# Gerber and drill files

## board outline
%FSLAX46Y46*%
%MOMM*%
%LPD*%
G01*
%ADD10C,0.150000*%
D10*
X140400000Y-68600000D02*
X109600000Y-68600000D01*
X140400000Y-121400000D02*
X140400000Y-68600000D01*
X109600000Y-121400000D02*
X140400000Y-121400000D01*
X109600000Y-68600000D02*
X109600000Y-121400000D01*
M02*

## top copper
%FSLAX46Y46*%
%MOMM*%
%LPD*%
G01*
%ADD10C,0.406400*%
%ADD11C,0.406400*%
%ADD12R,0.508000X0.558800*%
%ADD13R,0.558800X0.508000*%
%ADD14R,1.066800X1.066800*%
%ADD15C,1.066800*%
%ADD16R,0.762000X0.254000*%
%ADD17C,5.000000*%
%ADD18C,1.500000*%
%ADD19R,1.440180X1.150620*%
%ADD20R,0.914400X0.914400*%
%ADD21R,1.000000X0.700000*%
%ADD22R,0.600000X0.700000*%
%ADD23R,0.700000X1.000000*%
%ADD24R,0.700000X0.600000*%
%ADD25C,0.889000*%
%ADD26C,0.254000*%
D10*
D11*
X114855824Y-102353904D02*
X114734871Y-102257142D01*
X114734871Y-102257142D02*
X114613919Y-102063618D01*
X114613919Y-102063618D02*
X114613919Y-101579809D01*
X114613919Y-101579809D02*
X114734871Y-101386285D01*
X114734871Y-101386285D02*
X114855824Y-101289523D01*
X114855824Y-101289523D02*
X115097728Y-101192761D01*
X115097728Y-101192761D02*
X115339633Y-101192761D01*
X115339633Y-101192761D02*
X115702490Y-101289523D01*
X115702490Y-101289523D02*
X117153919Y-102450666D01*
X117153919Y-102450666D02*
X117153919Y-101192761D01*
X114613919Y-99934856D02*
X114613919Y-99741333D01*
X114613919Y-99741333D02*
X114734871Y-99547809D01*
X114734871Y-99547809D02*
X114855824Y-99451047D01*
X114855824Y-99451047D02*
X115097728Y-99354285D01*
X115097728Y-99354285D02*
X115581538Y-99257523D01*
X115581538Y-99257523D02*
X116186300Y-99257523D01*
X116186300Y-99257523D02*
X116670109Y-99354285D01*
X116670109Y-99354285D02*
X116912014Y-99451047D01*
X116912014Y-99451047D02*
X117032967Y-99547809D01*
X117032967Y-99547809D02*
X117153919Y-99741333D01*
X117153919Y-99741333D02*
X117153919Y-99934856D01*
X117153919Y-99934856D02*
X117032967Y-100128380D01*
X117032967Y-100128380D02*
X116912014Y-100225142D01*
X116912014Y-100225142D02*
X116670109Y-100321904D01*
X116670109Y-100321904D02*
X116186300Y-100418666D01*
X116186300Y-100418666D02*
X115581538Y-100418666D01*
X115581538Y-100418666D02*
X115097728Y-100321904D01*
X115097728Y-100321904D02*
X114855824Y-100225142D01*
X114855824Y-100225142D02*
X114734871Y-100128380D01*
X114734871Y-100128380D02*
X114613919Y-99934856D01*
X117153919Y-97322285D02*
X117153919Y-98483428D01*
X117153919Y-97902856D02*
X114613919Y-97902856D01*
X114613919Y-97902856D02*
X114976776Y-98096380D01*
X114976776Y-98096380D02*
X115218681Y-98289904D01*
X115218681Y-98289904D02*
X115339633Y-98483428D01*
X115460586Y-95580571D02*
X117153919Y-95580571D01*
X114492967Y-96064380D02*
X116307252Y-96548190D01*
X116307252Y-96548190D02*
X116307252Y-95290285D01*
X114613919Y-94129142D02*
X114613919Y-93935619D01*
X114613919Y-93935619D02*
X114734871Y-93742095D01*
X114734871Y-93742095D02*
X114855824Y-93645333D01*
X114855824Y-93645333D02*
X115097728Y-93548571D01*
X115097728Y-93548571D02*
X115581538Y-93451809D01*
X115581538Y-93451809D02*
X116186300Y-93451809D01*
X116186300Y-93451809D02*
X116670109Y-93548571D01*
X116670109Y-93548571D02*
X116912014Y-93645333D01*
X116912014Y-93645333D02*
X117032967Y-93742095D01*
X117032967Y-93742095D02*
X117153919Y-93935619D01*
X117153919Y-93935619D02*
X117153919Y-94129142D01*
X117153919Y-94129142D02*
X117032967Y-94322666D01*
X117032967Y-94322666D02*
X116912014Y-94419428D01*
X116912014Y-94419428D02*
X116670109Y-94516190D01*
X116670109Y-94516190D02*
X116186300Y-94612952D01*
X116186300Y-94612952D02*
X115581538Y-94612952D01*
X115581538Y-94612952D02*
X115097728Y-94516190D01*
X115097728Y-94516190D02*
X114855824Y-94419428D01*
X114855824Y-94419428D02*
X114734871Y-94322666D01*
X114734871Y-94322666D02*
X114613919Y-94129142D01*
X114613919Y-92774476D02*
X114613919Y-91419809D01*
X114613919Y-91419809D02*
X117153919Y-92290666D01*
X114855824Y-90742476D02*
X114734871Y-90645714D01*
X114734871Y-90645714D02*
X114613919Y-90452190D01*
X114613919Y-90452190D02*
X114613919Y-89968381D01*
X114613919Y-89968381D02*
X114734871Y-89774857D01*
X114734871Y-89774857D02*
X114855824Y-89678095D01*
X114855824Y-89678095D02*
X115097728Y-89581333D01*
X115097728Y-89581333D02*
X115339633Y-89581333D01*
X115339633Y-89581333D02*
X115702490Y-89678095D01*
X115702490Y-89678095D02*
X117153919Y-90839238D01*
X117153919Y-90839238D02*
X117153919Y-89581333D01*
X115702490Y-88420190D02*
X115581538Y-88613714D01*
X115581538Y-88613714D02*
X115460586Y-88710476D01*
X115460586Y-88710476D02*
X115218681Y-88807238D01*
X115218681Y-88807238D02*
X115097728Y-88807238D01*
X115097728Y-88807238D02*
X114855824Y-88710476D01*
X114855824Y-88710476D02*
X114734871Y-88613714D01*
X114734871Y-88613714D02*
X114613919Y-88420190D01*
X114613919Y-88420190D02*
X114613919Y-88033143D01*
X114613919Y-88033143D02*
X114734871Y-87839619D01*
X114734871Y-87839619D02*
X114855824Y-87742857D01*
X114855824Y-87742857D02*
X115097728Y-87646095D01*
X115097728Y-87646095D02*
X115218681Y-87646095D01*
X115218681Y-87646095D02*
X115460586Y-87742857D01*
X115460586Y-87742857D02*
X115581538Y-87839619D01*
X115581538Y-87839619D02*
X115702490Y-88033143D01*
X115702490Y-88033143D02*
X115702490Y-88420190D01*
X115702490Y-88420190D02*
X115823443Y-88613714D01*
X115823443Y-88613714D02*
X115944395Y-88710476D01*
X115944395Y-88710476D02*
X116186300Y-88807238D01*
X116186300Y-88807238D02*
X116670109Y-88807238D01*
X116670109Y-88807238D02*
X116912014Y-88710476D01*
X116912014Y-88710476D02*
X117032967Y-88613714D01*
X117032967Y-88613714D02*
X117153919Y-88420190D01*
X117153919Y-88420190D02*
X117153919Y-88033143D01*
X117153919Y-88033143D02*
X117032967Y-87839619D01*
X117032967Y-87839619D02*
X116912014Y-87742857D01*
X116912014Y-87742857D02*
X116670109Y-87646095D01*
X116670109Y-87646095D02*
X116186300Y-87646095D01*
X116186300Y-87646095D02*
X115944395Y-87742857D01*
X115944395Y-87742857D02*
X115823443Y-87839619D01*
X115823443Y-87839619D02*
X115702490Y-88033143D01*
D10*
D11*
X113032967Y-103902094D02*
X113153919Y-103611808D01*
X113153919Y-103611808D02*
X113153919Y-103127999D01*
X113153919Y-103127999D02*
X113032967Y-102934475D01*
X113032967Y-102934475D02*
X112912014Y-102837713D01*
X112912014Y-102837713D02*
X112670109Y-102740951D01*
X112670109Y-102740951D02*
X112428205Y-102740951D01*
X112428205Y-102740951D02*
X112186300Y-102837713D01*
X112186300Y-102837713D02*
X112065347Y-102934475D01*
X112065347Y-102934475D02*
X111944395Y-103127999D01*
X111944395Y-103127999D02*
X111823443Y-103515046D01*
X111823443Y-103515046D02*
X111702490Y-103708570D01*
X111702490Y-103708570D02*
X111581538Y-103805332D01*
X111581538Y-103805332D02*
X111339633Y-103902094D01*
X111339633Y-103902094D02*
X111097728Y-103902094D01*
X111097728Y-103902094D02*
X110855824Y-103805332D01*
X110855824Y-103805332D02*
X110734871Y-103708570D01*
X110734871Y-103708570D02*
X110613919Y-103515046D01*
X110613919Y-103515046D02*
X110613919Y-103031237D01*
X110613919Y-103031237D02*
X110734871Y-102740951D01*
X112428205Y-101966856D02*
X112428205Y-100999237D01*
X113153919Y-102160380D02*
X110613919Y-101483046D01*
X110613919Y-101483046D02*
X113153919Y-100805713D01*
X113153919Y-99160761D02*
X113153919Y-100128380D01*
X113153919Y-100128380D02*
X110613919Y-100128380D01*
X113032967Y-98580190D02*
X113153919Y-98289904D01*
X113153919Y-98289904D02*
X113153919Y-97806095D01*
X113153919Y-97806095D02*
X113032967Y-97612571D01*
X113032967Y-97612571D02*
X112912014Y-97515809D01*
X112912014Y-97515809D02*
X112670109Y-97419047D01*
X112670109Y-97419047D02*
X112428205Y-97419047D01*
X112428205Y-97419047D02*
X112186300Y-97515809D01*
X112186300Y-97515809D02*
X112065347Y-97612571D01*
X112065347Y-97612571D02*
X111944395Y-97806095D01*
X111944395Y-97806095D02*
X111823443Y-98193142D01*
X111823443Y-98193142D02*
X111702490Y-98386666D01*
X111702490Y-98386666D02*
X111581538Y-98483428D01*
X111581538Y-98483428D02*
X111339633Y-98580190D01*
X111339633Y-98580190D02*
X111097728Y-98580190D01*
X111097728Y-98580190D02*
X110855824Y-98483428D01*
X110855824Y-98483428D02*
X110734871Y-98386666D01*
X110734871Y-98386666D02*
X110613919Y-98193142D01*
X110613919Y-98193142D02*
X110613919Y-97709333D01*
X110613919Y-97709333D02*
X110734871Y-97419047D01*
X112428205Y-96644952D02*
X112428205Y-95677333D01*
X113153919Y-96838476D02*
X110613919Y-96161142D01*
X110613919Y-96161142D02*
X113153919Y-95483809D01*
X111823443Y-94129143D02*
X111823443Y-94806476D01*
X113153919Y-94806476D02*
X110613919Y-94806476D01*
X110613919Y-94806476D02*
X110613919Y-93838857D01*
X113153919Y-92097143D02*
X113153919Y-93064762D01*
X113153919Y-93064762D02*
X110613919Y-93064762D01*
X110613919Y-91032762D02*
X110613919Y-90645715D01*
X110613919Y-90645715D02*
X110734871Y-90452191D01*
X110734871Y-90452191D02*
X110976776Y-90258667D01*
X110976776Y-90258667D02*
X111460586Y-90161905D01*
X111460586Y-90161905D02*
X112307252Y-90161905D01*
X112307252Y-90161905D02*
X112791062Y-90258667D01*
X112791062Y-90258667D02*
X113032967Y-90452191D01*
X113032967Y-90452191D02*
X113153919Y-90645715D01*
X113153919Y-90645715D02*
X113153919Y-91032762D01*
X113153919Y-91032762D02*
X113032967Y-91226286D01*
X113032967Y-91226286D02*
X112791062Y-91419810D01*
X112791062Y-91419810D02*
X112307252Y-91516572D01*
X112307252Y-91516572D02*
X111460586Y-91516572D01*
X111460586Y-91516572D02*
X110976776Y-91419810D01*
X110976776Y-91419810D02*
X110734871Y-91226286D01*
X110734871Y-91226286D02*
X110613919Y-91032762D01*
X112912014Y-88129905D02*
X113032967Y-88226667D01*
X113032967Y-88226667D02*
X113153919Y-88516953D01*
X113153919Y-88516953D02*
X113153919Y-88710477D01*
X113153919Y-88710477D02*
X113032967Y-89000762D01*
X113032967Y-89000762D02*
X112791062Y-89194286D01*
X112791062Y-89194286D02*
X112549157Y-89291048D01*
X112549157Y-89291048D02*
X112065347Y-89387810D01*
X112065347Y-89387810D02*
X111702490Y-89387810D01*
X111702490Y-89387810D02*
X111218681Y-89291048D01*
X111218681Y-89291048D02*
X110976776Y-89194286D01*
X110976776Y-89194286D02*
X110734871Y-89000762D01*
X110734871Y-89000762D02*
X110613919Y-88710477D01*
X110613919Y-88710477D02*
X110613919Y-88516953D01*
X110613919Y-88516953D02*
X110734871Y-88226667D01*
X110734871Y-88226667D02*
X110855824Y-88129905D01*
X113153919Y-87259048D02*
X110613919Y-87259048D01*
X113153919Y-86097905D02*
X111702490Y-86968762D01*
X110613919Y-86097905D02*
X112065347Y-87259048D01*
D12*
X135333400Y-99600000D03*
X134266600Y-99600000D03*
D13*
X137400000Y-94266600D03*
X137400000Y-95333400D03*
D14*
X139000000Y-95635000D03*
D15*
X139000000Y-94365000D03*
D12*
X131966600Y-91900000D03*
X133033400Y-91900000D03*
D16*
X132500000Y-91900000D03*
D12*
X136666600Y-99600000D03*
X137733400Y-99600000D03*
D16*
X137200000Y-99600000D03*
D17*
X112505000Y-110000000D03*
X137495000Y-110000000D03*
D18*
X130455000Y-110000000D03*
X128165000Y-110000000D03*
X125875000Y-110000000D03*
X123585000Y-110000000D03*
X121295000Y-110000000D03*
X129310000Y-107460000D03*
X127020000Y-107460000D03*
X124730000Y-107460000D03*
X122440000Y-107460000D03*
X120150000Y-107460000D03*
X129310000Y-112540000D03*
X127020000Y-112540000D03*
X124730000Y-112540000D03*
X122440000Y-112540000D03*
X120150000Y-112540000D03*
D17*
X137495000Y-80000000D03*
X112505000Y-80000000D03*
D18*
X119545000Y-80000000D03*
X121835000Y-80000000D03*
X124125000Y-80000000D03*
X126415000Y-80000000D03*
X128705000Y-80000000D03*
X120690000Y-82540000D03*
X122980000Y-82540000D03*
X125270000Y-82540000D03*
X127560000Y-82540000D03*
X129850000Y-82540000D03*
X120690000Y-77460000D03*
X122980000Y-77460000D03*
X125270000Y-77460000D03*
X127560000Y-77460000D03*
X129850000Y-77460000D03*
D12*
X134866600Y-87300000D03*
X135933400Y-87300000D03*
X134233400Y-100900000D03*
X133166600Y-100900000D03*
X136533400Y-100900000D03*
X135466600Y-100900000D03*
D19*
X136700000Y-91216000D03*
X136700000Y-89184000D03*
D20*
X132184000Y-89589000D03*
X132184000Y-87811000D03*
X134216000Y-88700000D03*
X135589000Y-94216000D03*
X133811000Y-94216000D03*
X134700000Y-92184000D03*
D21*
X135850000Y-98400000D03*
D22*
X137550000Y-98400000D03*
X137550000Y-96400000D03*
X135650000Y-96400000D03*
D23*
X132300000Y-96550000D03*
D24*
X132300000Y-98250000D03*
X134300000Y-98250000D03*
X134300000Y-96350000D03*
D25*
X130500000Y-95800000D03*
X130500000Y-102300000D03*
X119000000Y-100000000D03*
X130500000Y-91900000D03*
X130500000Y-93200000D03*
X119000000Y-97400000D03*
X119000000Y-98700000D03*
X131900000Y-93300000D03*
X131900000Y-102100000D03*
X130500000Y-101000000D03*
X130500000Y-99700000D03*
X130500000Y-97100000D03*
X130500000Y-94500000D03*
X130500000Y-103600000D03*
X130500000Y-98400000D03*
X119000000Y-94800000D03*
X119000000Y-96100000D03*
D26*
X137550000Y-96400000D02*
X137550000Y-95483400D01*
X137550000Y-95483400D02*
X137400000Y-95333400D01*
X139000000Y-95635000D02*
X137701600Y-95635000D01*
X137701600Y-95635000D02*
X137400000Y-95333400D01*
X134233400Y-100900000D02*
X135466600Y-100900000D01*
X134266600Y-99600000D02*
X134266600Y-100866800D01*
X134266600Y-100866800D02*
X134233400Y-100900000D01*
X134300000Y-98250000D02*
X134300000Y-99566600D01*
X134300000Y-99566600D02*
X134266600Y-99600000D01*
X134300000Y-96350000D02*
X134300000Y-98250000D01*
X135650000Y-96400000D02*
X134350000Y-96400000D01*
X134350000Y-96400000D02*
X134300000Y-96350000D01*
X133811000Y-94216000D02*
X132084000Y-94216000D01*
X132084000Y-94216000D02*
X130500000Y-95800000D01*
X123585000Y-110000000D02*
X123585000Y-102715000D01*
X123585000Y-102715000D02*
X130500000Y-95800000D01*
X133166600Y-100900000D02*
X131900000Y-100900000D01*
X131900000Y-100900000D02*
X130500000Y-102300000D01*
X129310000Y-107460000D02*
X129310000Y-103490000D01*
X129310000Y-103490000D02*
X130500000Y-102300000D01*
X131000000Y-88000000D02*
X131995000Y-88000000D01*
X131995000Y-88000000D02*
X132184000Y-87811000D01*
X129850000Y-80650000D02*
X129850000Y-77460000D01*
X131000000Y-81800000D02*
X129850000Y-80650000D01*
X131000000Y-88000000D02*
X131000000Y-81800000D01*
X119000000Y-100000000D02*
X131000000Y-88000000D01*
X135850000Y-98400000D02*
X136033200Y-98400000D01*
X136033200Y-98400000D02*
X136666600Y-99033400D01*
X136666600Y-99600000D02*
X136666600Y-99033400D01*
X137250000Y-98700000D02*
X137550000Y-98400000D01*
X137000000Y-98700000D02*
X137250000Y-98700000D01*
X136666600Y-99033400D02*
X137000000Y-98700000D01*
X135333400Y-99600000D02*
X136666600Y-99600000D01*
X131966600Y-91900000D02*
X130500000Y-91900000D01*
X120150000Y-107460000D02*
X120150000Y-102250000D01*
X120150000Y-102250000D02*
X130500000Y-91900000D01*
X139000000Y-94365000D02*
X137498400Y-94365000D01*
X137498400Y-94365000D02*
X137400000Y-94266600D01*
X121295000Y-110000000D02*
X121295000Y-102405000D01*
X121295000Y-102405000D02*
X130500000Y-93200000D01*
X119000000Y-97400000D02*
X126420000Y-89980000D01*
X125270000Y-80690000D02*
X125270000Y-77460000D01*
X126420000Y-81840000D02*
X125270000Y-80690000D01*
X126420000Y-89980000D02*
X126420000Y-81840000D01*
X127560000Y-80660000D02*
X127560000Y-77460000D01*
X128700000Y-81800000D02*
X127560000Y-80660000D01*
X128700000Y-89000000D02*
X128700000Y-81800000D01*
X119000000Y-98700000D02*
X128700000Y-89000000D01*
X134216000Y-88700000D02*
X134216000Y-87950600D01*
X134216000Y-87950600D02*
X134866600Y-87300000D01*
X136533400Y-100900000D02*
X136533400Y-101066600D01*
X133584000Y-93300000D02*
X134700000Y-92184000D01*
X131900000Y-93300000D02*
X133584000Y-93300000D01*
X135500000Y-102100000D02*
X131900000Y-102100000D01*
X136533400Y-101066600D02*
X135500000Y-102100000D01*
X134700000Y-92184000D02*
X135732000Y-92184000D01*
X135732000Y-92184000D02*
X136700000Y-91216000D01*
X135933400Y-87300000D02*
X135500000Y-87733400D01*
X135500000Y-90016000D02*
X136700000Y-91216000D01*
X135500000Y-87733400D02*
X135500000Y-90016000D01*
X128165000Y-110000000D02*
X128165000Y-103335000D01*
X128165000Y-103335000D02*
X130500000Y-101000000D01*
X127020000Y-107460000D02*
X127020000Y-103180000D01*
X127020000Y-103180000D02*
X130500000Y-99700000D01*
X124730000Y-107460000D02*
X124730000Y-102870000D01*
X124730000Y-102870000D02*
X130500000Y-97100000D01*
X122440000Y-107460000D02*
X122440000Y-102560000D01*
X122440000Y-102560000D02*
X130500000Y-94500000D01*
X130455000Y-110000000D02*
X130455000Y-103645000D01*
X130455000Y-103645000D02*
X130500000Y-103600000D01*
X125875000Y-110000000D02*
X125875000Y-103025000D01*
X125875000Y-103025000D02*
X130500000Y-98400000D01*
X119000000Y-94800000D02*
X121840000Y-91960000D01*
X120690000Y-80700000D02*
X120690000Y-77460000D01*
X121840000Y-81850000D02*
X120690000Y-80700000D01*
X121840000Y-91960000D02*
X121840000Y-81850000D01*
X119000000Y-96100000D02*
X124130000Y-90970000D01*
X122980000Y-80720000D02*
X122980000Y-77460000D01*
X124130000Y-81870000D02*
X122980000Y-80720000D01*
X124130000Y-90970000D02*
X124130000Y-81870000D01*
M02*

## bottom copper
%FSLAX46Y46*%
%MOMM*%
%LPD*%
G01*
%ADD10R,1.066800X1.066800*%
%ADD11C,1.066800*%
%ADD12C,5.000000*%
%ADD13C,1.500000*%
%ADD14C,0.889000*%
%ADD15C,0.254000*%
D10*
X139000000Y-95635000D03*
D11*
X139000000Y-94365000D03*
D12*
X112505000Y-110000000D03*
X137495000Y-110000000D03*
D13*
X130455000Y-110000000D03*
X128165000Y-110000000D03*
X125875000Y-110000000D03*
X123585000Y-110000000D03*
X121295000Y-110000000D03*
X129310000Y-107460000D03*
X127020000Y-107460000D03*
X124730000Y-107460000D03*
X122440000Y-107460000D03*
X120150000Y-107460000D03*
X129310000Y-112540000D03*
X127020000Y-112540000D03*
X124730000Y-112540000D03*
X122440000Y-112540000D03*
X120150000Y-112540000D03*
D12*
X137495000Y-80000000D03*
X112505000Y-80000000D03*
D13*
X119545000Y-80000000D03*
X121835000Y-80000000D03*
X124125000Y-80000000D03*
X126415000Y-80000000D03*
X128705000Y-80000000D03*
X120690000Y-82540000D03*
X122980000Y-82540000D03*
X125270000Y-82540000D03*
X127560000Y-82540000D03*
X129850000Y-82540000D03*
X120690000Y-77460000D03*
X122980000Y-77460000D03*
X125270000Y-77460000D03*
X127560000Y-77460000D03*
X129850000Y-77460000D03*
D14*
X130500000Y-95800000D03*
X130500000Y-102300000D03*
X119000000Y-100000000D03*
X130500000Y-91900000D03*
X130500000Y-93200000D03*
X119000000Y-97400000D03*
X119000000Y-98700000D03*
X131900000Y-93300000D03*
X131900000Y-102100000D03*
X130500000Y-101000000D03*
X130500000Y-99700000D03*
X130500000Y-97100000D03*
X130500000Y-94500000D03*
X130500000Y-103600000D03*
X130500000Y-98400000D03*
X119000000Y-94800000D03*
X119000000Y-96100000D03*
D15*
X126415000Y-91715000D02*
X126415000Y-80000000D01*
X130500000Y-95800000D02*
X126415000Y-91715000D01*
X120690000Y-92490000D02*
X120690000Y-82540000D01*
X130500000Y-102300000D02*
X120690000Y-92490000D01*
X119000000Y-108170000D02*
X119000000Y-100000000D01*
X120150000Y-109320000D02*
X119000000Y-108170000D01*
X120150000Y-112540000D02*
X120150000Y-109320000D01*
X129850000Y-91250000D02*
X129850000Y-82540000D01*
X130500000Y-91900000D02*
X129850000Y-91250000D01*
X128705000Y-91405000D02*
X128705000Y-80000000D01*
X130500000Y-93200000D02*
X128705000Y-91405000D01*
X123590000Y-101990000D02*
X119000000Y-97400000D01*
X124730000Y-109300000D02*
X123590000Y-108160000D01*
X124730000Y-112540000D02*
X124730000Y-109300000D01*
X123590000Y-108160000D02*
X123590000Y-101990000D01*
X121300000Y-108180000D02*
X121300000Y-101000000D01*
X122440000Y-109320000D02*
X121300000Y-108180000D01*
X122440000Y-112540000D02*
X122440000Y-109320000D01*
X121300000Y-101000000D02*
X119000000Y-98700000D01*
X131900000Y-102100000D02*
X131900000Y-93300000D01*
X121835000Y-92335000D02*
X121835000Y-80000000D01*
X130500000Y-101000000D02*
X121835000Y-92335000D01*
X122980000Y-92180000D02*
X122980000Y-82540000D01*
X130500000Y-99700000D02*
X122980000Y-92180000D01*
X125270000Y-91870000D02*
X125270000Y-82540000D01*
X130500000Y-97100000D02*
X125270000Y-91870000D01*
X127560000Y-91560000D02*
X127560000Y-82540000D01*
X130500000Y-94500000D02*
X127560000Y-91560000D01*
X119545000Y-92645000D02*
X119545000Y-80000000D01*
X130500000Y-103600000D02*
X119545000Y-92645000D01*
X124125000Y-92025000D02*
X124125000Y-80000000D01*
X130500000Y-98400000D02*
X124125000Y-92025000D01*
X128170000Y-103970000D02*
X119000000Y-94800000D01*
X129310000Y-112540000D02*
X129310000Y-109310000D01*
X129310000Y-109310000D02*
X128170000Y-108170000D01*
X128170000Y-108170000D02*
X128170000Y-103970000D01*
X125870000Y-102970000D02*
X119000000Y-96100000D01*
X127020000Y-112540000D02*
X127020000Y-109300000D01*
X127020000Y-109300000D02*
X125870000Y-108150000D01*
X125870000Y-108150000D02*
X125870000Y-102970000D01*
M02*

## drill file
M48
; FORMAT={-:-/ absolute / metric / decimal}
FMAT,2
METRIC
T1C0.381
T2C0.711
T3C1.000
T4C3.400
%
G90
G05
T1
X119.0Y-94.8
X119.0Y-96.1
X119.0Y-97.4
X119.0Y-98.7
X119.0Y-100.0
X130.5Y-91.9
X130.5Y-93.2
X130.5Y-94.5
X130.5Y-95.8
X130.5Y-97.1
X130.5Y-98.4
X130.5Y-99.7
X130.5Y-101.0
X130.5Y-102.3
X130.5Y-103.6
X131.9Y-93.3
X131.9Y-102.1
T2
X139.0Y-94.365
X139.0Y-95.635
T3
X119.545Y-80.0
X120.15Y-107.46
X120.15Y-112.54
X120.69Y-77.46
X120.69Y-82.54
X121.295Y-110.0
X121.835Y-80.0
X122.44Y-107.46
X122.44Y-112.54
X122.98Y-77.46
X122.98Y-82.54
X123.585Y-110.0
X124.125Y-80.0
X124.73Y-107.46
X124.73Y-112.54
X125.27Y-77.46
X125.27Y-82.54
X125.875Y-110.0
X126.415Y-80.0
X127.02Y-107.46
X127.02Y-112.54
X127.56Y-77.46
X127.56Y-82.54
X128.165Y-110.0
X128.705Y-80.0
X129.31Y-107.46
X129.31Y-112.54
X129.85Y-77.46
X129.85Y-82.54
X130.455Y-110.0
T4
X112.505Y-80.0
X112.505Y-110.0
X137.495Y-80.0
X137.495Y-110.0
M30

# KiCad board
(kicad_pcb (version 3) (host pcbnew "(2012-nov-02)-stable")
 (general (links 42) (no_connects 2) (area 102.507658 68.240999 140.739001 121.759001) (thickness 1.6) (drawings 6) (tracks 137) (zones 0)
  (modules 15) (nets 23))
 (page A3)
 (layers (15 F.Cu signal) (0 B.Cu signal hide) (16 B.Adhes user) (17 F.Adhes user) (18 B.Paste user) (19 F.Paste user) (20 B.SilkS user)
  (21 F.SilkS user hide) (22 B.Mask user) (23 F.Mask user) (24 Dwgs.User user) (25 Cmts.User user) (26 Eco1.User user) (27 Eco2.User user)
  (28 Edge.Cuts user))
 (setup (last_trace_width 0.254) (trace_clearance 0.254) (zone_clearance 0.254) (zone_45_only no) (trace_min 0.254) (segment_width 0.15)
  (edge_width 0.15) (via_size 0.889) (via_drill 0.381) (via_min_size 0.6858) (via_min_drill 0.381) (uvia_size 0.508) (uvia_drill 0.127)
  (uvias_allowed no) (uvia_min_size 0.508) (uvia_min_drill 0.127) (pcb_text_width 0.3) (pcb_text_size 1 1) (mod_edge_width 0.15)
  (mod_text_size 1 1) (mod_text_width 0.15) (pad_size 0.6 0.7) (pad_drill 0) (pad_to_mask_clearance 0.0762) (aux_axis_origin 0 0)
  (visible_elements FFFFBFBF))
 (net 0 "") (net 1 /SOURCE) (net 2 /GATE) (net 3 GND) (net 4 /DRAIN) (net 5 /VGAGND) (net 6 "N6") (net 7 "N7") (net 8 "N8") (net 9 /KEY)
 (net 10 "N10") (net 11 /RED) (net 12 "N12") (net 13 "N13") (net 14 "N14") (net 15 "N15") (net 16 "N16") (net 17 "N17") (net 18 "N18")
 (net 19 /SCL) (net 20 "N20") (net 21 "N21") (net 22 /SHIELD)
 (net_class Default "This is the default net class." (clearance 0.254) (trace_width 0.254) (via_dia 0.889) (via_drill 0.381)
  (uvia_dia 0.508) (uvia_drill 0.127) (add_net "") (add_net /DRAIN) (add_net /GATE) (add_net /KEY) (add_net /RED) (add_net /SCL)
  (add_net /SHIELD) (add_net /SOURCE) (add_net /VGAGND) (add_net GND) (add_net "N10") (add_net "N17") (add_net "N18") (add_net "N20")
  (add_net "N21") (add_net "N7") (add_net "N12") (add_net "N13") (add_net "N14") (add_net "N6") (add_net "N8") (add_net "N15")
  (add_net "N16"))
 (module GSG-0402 (layer F.Cu) (at 134.8 99.6) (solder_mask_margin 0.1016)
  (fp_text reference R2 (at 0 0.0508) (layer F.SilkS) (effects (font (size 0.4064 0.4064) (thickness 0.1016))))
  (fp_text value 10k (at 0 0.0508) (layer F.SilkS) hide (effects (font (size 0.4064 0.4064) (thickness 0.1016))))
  (pad 2 smd rect (at 0.5334 0) (size 0.508 0.5588) (layers F.Cu F.Paste F.Mask) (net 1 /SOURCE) (solder_mask_margin 0.1016))
  (pad 1 smd rect (at -0.5334 0) (size 0.508 0.5588) (layers F.Cu F.Paste F.Mask) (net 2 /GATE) (die_length -2147.483648)
   (solder_mask_margin 0.1016)))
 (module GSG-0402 (layer F.Cu) (at 137.4 94.8 90) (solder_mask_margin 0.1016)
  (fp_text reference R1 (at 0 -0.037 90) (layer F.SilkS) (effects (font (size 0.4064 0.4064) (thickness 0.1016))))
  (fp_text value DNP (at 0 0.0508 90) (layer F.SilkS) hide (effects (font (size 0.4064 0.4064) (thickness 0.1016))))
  (pad 2 smd rect (at 0.5334 0 90) (size 0.508 0.5588) (layers F.Cu F.Paste F.Mask) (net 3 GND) (solder_mask_margin 0.1016))
  (pad 1 smd rect (at -0.5334 0 90) (size 0.508 0.5588) (layers F.Cu F.Paste F.Mask) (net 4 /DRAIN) (die_length -2147.483648)
   (solder_mask_margin 0.1016)))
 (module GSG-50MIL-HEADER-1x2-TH (layer F.Cu) (at 139 95 90)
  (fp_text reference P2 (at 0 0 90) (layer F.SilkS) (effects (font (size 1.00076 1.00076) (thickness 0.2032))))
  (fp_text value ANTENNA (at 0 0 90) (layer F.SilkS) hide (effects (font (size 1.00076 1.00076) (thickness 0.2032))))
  (pad 1 thru_hole rect (at -0.635 0 90) (size 1.0668 1.0668) (drill 0.7112) (layers *.Cu *.Mask) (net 4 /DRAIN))
  (pad 2 thru_hole circle (at 0.635 0 90) (size 1.0668 1.0668) (drill 0.7112) (layers *.Cu *.Mask) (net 3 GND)))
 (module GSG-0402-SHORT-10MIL (layer F.Cu) (at 132.5 91.9 180) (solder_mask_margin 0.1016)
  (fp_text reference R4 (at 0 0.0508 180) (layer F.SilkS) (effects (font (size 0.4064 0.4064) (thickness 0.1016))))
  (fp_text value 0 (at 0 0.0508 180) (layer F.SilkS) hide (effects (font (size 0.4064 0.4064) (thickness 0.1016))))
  (pad 2 smd rect (at 0.5334 0 180) (size 0.508 0.5588) (layers F.Cu F.Mask) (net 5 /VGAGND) (solder_mask_margin 0.1016))
  (pad 1 smd rect (at -0.5334 0 180) (size 0.508 0.5588) (layers F.Cu F.Mask) (die_length -2147.483648) (solder_mask_margin 0.1016))
  (pad "" smd rect (at 0 0 180) (size 0.762 0.254) (layers F.Cu F.Mask)))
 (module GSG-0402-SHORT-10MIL (layer F.Cu) (at 137.2 99.6 180) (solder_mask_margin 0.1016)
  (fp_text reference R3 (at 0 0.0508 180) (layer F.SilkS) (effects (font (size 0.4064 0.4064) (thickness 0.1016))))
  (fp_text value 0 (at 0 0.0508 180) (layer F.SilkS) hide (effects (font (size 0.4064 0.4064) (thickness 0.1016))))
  (pad 2 smd rect (at 0.5334 0 180) (size 0.508 0.5588) (layers F.Cu F.Mask) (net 1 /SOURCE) (solder_mask_margin 0.1016))
  (pad 1 smd rect (at -0.5334 0 180) (size 0.508 0.5588) (layers F.Cu F.Mask) (die_length -2147.483648) (solder_mask_margin 0.1016))
  (pad "" smd rect (at 0 0 180) (size 0.762 0.254) (layers F.Cu F.Mask)))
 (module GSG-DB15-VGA (layer F.Cu) (at 125 110)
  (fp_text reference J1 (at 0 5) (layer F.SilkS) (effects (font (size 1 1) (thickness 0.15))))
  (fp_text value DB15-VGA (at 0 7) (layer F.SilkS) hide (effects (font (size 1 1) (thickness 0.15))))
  (pad 0 thru_hole circle (at -12.495 0) (size 5 5) (drill 3.4) (layers *.Cu *.Mask))
  (pad 0 thru_hole circle (at 12.495 0) (size 5 5) (drill 3.4) (layers *.Cu *.Mask))
  (pad 6 thru_hole circle (at 5.455 0) (size 1.5 1.5) (drill 1) (layers *.Cu *.Mask) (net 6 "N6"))
  (pad 7 thru_hole circle (at 3.165 0) (size 1.5 1.5) (drill 1) (layers *.Cu *.Mask) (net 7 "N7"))
  (pad 8 thru_hole circle (at 0.875 0) (size 1.5 1.5) (drill 1) (layers *.Cu *.Mask) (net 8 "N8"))
  (pad 9 thru_hole circle (at -1.415 0) (size 1.5 1.5) (drill 1) (layers *.Cu *.Mask) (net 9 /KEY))
  (pad 10 thru_hole circle (at -3.705 0) (size 1.5 1.5) (drill 1) (layers *.Cu *.Mask) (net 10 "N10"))
  (pad 1 thru_hole circle (at 4.31 -2.54) (size 1.5 1.5) (drill 1) (layers *.Cu *.Mask) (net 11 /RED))
  (pad 2 thru_hole circle (at 2.02 -2.54) (size 1.5 1.5) (drill 1) (layers *.Cu *.Mask) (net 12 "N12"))
  (pad 3 thru_hole circle (at -0.27 -2.54) (size 1.5 1.5) (drill 1) (layers *.Cu *.Mask) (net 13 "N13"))
  (pad 4 thru_hole circle (at -2.56 -2.54) (size 1.5 1.5) (drill 1) (layers *.Cu *.Mask) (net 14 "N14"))
  (pad 5 thru_hole circle (at -4.85 -2.54) (size 1.5 1.5) (drill 1) (layers *.Cu *.Mask) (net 5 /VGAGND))
  (pad 11 thru_hole circle (at 4.31 2.54) (size 1.5 1.5) (drill 1) (layers *.Cu *.Mask) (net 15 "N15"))
  (pad 12 thru_hole circle (at 2.02 2.54) (size 1.5 1.5) (drill 1) (layers *.Cu *.Mask) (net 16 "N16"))
  (pad 13 thru_hole circle (at -0.27 2.54) (size 1.5 1.5) (drill 1) (layers *.Cu *.Mask) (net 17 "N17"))
  (pad 14 thru_hole circle (at -2.56 2.54) (size 1.5 1.5) (drill 1) (layers *.Cu *.Mask) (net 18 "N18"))
  (pad 15 thru_hole circle (at -4.85 2.54) (size 1.5 1.5) (drill 1) (layers *.Cu *.Mask) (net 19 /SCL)))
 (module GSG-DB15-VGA (layer F.Cu) (at 125 80 180)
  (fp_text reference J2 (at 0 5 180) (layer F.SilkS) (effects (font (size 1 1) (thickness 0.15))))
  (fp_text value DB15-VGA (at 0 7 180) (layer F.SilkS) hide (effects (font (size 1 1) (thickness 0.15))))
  (pad 0 thru_hole circle (at -12.495 0 180) (size 5 5) (drill 3.4) (layers *.Cu *.Mask))
  (pad 0 thru_hole circle (at 12.495 0 180) (size 5 5) (drill 3.4) (layers *.Cu *.Mask))
  (pad 6 thru_hole circle (at 5.455 0 180) (size 1.5 1.5) (drill 1) (layers *.Cu *.Mask) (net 6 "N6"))
  (pad 7 thru_hole circle (at 3.165 0 180) (size 1.5 1.5) (drill 1) (layers *.Cu *.Mask) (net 7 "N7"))
  (pad 8 thru_hole circle (at 0.875 0 180) (size 1.5 1.5) (drill 1) (layers *.Cu *.Mask) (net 8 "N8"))
  (pad 9 thru_hole circle (at -1.415 0 180) (size 1.5 1.5) (drill 1) (layers *.Cu *.Mask) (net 9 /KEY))
  (pad 10 thru_hole circle (at -3.705 0 180) (size 1.5 1.5) (drill 1) (layers *.Cu *.Mask) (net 10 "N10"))
  (pad 1 thru_hole circle (at 4.31 -2.54 180) (size 1.5 1.5) (drill 1) (layers *.Cu *.Mask) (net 11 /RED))
  (pad 2 thru_hole circle (at 2.02 -2.54 180) (size 1.5 1.5) (drill 1) (layers *.Cu *.Mask) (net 12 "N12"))
  (pad 3 thru_hole circle (at -0.27 -2.54 180) (size 1.5 1.5) (drill 1) (layers *.Cu *.Mask) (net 13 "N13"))
  (pad 4 thru_hole circle (at -2.56 -2.54 180) (size 1.5 1.5) (drill 1) (layers *.Cu *.Mask) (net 14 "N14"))
  (pad 5 thru_hole circle (at -4.85 -2.54 180) (size 1.5 1.5) (drill 1) (layers *.Cu *.Mask) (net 5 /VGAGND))
  (pad 11 thru_hole circle (at 4.31 2.54 180) (size 1.5 1.5) (drill 1) (layers *.Cu *.Mask) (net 15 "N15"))
  (pad 12 thru_hole circle (at 2.02 2.54 180) (size 1.5 1.5) (drill 1) (layers *.Cu *.Mask) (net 16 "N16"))
  (pad 13 thru_hole circle (at -0.27 2.54 180) (size 1.5 1.5) (drill 1) (layers *.Cu *.Mask) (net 17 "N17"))
  (pad 14 thru_hole circle (at -2.56 2.54 180) (size 1.5 1.5) (drill 1) (layers *.Cu *.Mask) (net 18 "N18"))
  (pad 15 thru_hole circle (at -4.85 2.54 180) (size 1.5 1.5) (drill 1) (layers *.Cu *.Mask) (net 19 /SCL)))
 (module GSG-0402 (layer F.Cu) (at 135.4 87.3 180) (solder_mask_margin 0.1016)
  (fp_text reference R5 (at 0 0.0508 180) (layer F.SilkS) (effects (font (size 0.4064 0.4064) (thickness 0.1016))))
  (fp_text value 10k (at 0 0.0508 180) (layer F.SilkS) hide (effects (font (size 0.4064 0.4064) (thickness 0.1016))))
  (pad 2 smd rect (at 0.5334 0 180) (size 0.508 0.5588) (layers F.Cu F.Paste F.Mask) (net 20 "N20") (solder_mask_margin 0.1016))
  (pad 1 smd rect (at -0.5334 0 180) (size 0.508 0.5588) (layers F.Cu F.Paste F.Mask) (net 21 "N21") (die_length -2147.483648)
   (solder_mask_margin 0.1016)))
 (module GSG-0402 (layer F.Cu) (at 133.7 100.9) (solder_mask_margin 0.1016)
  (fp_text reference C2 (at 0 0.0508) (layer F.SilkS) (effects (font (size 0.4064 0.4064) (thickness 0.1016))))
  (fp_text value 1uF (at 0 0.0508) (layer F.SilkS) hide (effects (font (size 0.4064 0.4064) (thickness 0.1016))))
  (pad 2 smd rect (at 0.5334 0) (size 0.508 0.5588) (layers F.Cu F.Paste F.Mask) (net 2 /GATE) (solder_mask_margin 0.1016))
  (pad 1 smd rect (at -0.5334 0) (size 0.508 0.5588) (layers F.Cu F.Paste F.Mask) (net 11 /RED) (die_length -2147.483648)
   (solder_mask_margin 0.1016)))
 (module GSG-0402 (layer F.Cu) (at 136 100.9) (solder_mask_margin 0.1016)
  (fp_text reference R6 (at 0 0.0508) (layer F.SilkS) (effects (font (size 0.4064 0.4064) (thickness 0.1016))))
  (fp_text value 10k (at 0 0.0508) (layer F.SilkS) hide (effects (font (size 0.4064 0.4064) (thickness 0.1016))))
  (pad 2 smd rect (at 0.5334 0) (size 0.508 0.5588) (layers F.Cu F.Paste F.Mask) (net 21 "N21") (solder_mask_margin 0.1016))
  (pad 1 smd rect (at -0.5334 0) (size 0.508 0.5588) (layers F.Cu F.Paste F.Mask) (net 2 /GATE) (die_length -2147.483648)
   (solder_mask_margin 0.1016)))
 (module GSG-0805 (layer F.Cu) (at 136.7 90.2 270) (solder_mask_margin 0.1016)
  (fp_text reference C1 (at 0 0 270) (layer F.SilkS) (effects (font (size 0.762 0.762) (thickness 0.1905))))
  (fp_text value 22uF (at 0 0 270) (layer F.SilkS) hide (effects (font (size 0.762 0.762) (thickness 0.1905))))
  (pad 2 smd rect (at 1.016 0 270) (size 1.15062 1.44018) (layers F.Cu F.Paste F.Mask) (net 21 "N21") (die_length 0.08128)
   (solder_mask_margin 0.1016) (clearance 0.1778))
  (pad 1 smd rect (at -1.016 0 270) (size 1.15062 1.44018) (layers F.Cu F.Paste F.Mask) (die_length -2147.483648)
   (solder_mask_margin 0.1016) (clearance 0.1778)))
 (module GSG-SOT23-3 (layer F.Cu) (at 133.2 88.7 90)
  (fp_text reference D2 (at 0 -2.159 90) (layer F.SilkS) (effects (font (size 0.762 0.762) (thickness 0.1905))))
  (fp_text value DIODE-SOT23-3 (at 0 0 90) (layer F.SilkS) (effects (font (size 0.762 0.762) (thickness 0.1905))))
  (pad 2 smd rect (at -0.889 -1.016 90) (size 0.9144 0.9144) (layers F.Cu F.Paste F.Mask) (die_length 0.00762))
  (pad 1 smd rect (at 0.889 -1.016 90) (size 0.9144 0.9144) (layers F.Cu F.Paste F.Mask) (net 19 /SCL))
  (pad 3 smd rect (at 0 1.016 90) (size 0.9144 0.9144) (layers F.Cu F.Paste F.Mask) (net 20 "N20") (die_length 0.28194)))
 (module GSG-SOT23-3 (layer F.Cu) (at 134.7 93.2 180)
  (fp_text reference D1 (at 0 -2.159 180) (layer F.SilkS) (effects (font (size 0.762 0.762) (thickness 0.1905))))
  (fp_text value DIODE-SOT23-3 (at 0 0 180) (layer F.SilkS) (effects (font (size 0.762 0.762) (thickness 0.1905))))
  (pad 2 smd rect (at -0.889 -1.016 180) (size 0.9144 0.9144) (layers F.Cu F.Paste F.Mask) (die_length 0.00762))
  (pad 1 smd rect (at 0.889 -1.016 180) (size 0.9144 0.9144) (layers F.Cu F.Paste F.Mask) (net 9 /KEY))
  (pad 3 smd rect (at 0 1.016 180) (size 0.9144 0.9144) (layers F.Cu F.Paste F.Mask) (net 21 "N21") (die_length 0.28194)))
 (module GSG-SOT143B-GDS (layer F.Cu) (at 136.6 97.4)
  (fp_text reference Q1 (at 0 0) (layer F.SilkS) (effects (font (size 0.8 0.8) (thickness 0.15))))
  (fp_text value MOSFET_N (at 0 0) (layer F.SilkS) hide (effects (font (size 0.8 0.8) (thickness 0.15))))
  (pad B smd rect (at -0.75 1) (size 1 0.7) (layers F.Cu F.Paste F.Mask) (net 1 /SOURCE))
  (pad S smd rect (at 0.95 1) (size 0.6 0.7) (layers F.Cu F.Paste F.Mask) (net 1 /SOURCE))
  (pad D smd rect (at 0.95 -1) (size 0.6 0.7) (layers F.Cu F.Paste F.Mask) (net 4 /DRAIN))
  (pad G smd rect (at -0.95 -1) (size 0.6 0.7) (layers F.Cu F.Paste F.Mask) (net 2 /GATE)))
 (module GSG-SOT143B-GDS (layer F.Cu) (at 133.3 97.3 270)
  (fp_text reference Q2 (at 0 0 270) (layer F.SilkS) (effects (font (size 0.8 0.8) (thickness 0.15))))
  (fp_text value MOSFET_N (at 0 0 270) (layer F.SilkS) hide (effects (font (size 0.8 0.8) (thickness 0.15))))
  (pad B smd rect (at -0.75 1 270) (size 1 0.7) (layers F.Cu F.Paste F.Mask))
  (pad S smd rect (at 0.95 1 270) (size 0.6 0.7) (layers F.Cu F.Paste F.Mask))
  (pad D smd rect (at 0.95 -1 270) (size 0.6 0.7) (layers F.Cu F.Paste F.Mask) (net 2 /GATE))
  (pad G smd rect (at -0.95 -1 270) (size 0.6 0.7) (layers F.Cu F.Paste F.Mask) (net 2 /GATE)))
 (gr_line (start 140.4 68.6) (end 109.6 68.6) (angle 90) (layer Edge.Cuts) (width 0.15))
 (gr_line (start 140.4 121.4) (end 140.4 68.6) (angle 90) (layer Edge.Cuts) (width 0.15))
 (gr_line (start 109.6 121.4) (end 140.4 121.4) (angle 90) (layer Edge.Cuts) (width 0.15))
 (gr_line (start 109.6 68.6) (end 109.6 121.4) (angle 90) (layer Edge.Cuts) (width 0.15))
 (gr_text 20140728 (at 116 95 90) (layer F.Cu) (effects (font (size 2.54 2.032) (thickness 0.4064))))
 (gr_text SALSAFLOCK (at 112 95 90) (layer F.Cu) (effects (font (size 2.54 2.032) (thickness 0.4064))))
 (segment (start 137.55 96.4) (end 137.55 95.4834) (width 0.254) (layer F.Cu) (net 4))
 (segment (start 137.55 95.4834) (end 137.4 95.3334) (width 0.254) (layer F.Cu) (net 4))
 (segment (start 139 95.635) (end 137.7016 95.635) (width 0.254) (layer F.Cu) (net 4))
 (segment (start 137.7016 95.635) (end 137.4 95.3334) (width 0.254) (layer F.Cu) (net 4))
 (segment (start 134.2334 100.9) (end 135.4666 100.9) (width 0.254) (layer F.Cu) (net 2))
 (segment (start 134.2666 99.6) (end 134.2666 100.8668) (width 0.254) (layer F.Cu) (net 2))
 (segment (start 134.2666 100.8668) (end 134.2334 100.9) (width 0.254) (layer F.Cu) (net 2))
 (segment (start 134.3 98.25) (end 134.3 99.5666) (width 0.254) (layer F.Cu) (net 2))
 (segment (start 134.3 99.5666) (end 134.2666 99.6) (width 0.254) (layer F.Cu) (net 2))
 (segment (start 134.3 96.35) (end 134.3 98.25) (width 0.254) (layer F.Cu) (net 2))
 (segment (start 135.65 96.4) (end 134.35 96.4) (width 0.254) (layer F.Cu) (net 2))
 (segment (start 134.35 96.4) (end 134.3 96.35) (width 0.254) (layer F.Cu) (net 2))
 (segment (start 133.811 94.216) (end 132.084 94.216) (width 0.254) (layer F.Cu) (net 9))
 (segment (start 132.084 94.216) (end 130.5 95.8) (width 0.254) (layer F.Cu) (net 9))
 (segment (start 123.585 110) (end 123.585 102.715) (width 0.254) (layer F.Cu) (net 9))
 (segment (start 126.415 91.715) (end 126.415 80) (width 0.254) (layer B.Cu) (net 9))
 (segment (start 130.5 95.8) (end 126.415 91.715) (width 0.254) (layer B.Cu) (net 9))
 (segment (start 123.585 102.715) (end 130.5 95.8) (width 0.254) (layer F.Cu) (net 9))
 (segment (start 133.1666 100.9) (end 131.9 100.9) (width 0.254) (layer F.Cu) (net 11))
 (segment (start 131.9 100.9) (end 130.5 102.3) (width 0.254) (layer F.Cu) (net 11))
 (segment (start 129.31 107.46) (end 129.31 103.49) (width 0.254) (layer F.Cu) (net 11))
 (segment (start 120.69 92.49) (end 120.69 82.54) (width 0.254) (layer B.Cu) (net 11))
 (segment (start 130.5 102.3) (end 120.69 92.49) (width 0.254) (layer B.Cu) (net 11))
 (segment (start 129.31 103.49) (end 130.5 102.3) (width 0.254) (layer F.Cu) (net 11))
 (segment (start 131 88) (end 131.995 88) (width 0.254) (layer F.Cu) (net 19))
 (segment (start 131.995 88) (end 132.184 87.811) (width 0.254) (layer F.Cu) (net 19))
 (segment (start 119 108.17) (end 119 100) (width 0.254) (layer B.Cu) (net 19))
 (segment (start 120.15 109.32) (end 119 108.17) (width 0.254) (layer B.Cu) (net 19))
 (segment (start 120.15 112.54) (end 120.15 109.32) (width 0.254) (layer B.Cu) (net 19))
 (segment (start 129.85 80.65) (end 129.85 77.46) (width 0.254) (layer F.Cu) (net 19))
 (segment (start 131 81.8) (end 129.85 80.65) (width 0.254) (layer F.Cu) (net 19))
 (segment (start 131 88) (end 131 81.8) (width 0.254) (layer F.Cu) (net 19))
 (segment (start 119 100) (end 131 88) (width 0.254) (layer F.Cu) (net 19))
 (segment (start 135.85 98.4) (end 136.0332 98.4) (width 0.254) (layer F.Cu) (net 1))
 (segment (start 136.0332 98.4) (end 136.6666 99.0334) (width 0.254) (layer F.Cu) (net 1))
 (segment (start 136.6666 99.6) (end 136.6666 99.0334) (width 0.254) (layer F.Cu) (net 1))
 (segment (start 137.25 98.7) (end 137.55 98.4) (width 0.254) (layer F.Cu) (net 1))
 (segment (start 137 98.7) (end 137.25 98.7) (width 0.254) (layer F.Cu) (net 1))
 (segment (start 136.6666 99.0334) (end 137 98.7) (width 0.254) (layer F.Cu) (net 1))
 (segment (start 135.3334 99.6) (end 136.6666 99.6) (width 0.254) (layer F.Cu) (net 1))
 (segment (start 131.9666 91.9) (end 130.5 91.9) (width 0.254) (layer F.Cu) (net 5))
 (segment (start 120.15 107.46) (end 120.15 102.25) (width 0.254) (layer F.Cu) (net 5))
 (segment (start 129.85 91.25) (end 129.85 82.54) (width 0.254) (layer B.Cu) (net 5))
 (segment (start 130.5 91.9) (end 129.85 91.25) (width 0.254) (layer B.Cu) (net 5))
 (segment (start 120.15 102.25) (end 130.5 91.9) (width 0.254) (layer F.Cu) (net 5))
 (segment (start 139 94.365) (end 137.4984 94.365) (width 0.254) (layer F.Cu) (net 3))
 (segment (start 137.4984 94.365) (end 137.4 94.2666) (width 0.254) (layer F.Cu) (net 3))
 (segment (start 121.295 110) (end 121.295 102.405) (width 0.254) (layer F.Cu) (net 10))
 (segment (start 128.705 91.405) (end 128.705 80) (width 0.254) (layer B.Cu) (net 10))
 (segment (start 130.5 93.2) (end 128.705 91.405) (width 0.254) (layer B.Cu) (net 10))
 (segment (start 121.295 102.405) (end 130.5 93.2) (width 0.254) (layer F.Cu) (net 10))
 (segment (start 119 97.4) (end 126.42 89.98) (width 0.254) (layer F.Cu) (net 17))
 (segment (start 123.59 101.99) (end 119 97.4) (width 0.254) (layer B.Cu) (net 17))
 (segment (start 124.73 109.3) (end 123.59 108.16) (width 0.254) (layer B.Cu) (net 17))
 (segment (start 124.73 112.54) (end 124.73 109.3) (width 0.254) (layer B.Cu) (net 17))
 (segment (start 123.59 108.16) (end 123.59 101.99) (width 0.254) (layer B.Cu) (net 17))
 (segment (start 125.27 80.69) (end 125.27 77.46) (width 0.254) (layer F.Cu) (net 17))
 (segment (start 126.42 81.84) (end 125.27 80.69) (width 0.254) (layer F.Cu) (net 17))
 (segment (start 126.42 89.98) (end 126.42 81.84) (width 0.254) (layer F.Cu) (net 17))
 (segment (start 121.3 108.18) (end 121.3 101) (width 0.254) (layer B.Cu) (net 18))
 (segment (start 122.44 109.32) (end 121.3 108.18) (width 0.254) (layer B.Cu) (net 18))
 (segment (start 122.44 112.54) (end 122.44 109.32) (width 0.254) (layer B.Cu) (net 18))
 (segment (start 127.56 80.66) (end 127.56 77.46) (width 0.254) (layer F.Cu) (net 18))
 (segment (start 128.7 81.8) (end 127.56 80.66) (width 0.254) (layer F.Cu) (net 18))
 (segment (start 128.7 89) (end 128.7 81.8) (width 0.254) (layer F.Cu) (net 18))
 (segment (start 119 98.7) (end 128.7 89) (width 0.254) (layer F.Cu) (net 18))
 (segment (start 121.3 101) (end 119 98.7) (width 0.254) (layer B.Cu) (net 18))
 (segment (start 134.216 88.7) (end 134.216 87.9506) (width 0.254) (layer F.Cu) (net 20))
 (segment (start 134.216 87.9506) (end 134.8666 87.3) (width 0.254) (layer F.Cu) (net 20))
 (segment (start 136.5334 100.9) (end 136.5334 101.0666) (width 0.254) (layer F.Cu) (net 21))
 (segment (start 133.584 93.3) (end 134.7 92.184) (width 0.254) (layer F.Cu) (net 21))
 (segment (start 131.9 93.3) (end 133.584 93.3) (width 0.254) (layer F.Cu) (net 21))
 (segment (start 131.9 102.1) (end 131.9 93.3) (width 0.254) (layer B.Cu) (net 21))
 (segment (start 135.5 102.1) (end 131.9 102.1) (width 0.254) (layer F.Cu) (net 21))
 (segment (start 136.5334 101.0666) (end 135.5 102.1) (width 0.254) (layer F.Cu) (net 21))
 (segment (start 134.7 92.184) (end 135.732 92.184) (width 0.254) (layer F.Cu) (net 21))
 (segment (start 135.732 92.184) (end 136.7 91.216) (width 0.254) (layer F.Cu) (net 21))
 (segment (start 135.9334 87.3) (end 135.5 87.7334) (width 0.254) (layer F.Cu) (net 21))
 (segment (start 135.5 90.016) (end 136.7 91.216) (width 0.254) (layer F.Cu) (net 21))
 (segment (start 135.5 87.7334) (end 135.5 90.016) (width 0.254) (layer F.Cu) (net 21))
 (segment (start 128.165 110) (end 128.165 103.335) (width 0.254) (layer F.Cu) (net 7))
 (segment (start 121.835 92.335) (end 121.835 80) (width 0.254) (layer B.Cu) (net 7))
 (segment (start 130.5 101) (end 121.835 92.335) (width 0.254) (layer B.Cu) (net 7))
 (segment (start 128.165 103.335) (end 130.5 101) (width 0.254) (layer F.Cu) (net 7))
 (segment (start 127.02 107.46) (end 127.02 103.18) (width 0.254) (layer F.Cu) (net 12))
 (segment (start 122.98 92.18) (end 122.98 82.54) (width 0.254) (layer B.Cu) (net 12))
 (segment (start 130.5 99.7) (end 122.98 92.18) (width 0.254) (layer B.Cu) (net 12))
 (segment (start 127.02 103.18) (end 130.5 99.7) (width 0.254) (layer F.Cu) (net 12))
 (segment (start 124.73 107.46) (end 124.73 102.87) (width 0.254) (layer F.Cu) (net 13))
 (segment (start 125.27 91.87) (end 125.27 82.54) (width 0.254) (layer B.Cu) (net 13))
 (segment (start 130.5 97.1) (end 125.27 91.87) (width 0.254) (layer B.Cu) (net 13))
 (segment (start 124.73 102.87) (end 130.5 97.1) (width 0.254) (layer F.Cu) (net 13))
 (segment (start 122.44 107.46) (end 122.44 102.56) (width 0.254) (layer F.Cu) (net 14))
 (segment (start 127.56 91.56) (end 127.56 82.54) (width 0.254) (layer B.Cu) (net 14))
 (segment (start 130.5 94.5) (end 127.56 91.56) (width 0.254) (layer B.Cu) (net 14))
 (segment (start 122.44 102.56) (end 130.5 94.5) (width 0.254) (layer F.Cu) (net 14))
 (segment (start 130.455 110) (end 130.455 103.645) (width 0.254) (layer F.Cu) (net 6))
 (segment (start 119.545 92.645) (end 119.545 80) (width 0.254) (layer B.Cu) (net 6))
 (segment (start 130.5 103.6) (end 119.545 92.645) (width 0.254) (layer B.Cu) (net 6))
 (segment (start 130.455 103.645) (end 130.5 103.6) (width 0.254) (layer F.Cu) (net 6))
 (segment (start 125.875 110) (end 125.875 103.025) (width 0.254) (layer F.Cu) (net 8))
 (segment (start 124.125 92.025) (end 124.125 80) (width 0.254) (layer B.Cu) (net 8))
 (segment (start 130.5 98.4) (end 124.125 92.025) (width 0.254) (layer B.Cu) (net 8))
 (segment (start 125.875 103.025) (end 130.5 98.4) (width 0.254) (layer F.Cu) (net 8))
 (segment (start 119 94.8) (end 121.84 91.96) (width 0.254) (layer F.Cu) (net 15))
 (segment (start 128.17 103.97) (end 119 94.8) (width 0.254) (layer B.Cu) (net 15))
 (segment (start 129.31 112.54) (end 129.31 109.31) (width 0.254) (layer B.Cu) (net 15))
 (segment (start 129.31 109.31) (end 128.17 108.17) (width 0.254) (layer B.Cu) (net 15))
 (segment (start 128.17 108.17) (end 128.17 103.97) (width 0.254) (layer B.Cu) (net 15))
 (segment (start 120.69 80.7) (end 120.69 77.46) (width 0.254) (layer F.Cu) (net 15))
 (segment (start 121.84 81.85) (end 120.69 80.7) (width 0.254) (layer F.Cu) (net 15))
 (segment (start 121.84 91.96) (end 121.84 81.85) (width 0.254) (layer F.Cu) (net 15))
 (segment (start 119 96.1) (end 124.13 90.97) (width 0.254) (layer F.Cu) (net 16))
 (segment (start 125.87 102.97) (end 119 96.1) (width 0.254) (layer B.Cu) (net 16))
 (segment (start 127.02 112.54) (end 127.02 109.3) (width 0.254) (layer B.Cu) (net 16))
 (segment (start 127.02 109.3) (end 125.87 108.15) (width 0.254) (layer B.Cu) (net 16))
 (segment (start 125.87 108.15) (end 125.87 102.97) (width 0.254) (layer B.Cu) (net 16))
 (segment (start 122.98 80.72) (end 122.98 77.46) (width 0.254) (layer F.Cu) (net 16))
 (segment (start 124.13 81.87) (end 122.98 80.72) (width 0.254) (layer F.Cu) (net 16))
 (segment (start 124.13 90.97) (end 124.13 81.87) (width 0.254) (layer F.Cu) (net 16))
 (via (at 130.5 95.8) (size 0.889) (layers F.Cu B.Cu) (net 9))
 (via (at 130.5 102.3) (size 0.889) (layers F.Cu B.Cu) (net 11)) (via (at 119 100) (size 0.889) (layers F.Cu B.Cu) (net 19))
 (via (at 130.5 91.9) (size 0.889) (layers F.Cu B.Cu) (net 5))
 (via (at 130.5 93.2) (size 0.889) (layers F.Cu B.Cu) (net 10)) (via (at 119 97.4) (size 0.889) (layers F.Cu B.Cu) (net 17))
 (via (at 119 98.7) (size 0.889) (layers F.Cu B.Cu) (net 18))
 (via (at 131.9 93.3) (size 0.889) (layers F.Cu B.Cu) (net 21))
 (via (at 131.9 102.1) (size 0.889) (layers F.Cu B.Cu) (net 21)) (via (at 130.5 101) (size 0.889) (layers F.Cu B.Cu) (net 7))
 (via (at 130.5 99.7) (size 0.889) (layers F.Cu B.Cu) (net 12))
 (via (at 130.5 97.1) (size 0.889) (layers F.Cu B.Cu) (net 13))
 (via (at 130.5 94.5) (size 0.889) (layers F.Cu B.Cu) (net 14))
 (via (at 130.5 103.6) (size 0.889) (layers F.Cu B.Cu) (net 6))
 (via (at 130.5 98.4) (size 0.889) (layers F.Cu B.Cu) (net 8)) (via (at 119 94.8) (size 0.889) (layers F.Cu B.Cu) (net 15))
 (via (at 119 96.1) (size 0.889) (layers F.Cu B.Cu) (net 16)))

